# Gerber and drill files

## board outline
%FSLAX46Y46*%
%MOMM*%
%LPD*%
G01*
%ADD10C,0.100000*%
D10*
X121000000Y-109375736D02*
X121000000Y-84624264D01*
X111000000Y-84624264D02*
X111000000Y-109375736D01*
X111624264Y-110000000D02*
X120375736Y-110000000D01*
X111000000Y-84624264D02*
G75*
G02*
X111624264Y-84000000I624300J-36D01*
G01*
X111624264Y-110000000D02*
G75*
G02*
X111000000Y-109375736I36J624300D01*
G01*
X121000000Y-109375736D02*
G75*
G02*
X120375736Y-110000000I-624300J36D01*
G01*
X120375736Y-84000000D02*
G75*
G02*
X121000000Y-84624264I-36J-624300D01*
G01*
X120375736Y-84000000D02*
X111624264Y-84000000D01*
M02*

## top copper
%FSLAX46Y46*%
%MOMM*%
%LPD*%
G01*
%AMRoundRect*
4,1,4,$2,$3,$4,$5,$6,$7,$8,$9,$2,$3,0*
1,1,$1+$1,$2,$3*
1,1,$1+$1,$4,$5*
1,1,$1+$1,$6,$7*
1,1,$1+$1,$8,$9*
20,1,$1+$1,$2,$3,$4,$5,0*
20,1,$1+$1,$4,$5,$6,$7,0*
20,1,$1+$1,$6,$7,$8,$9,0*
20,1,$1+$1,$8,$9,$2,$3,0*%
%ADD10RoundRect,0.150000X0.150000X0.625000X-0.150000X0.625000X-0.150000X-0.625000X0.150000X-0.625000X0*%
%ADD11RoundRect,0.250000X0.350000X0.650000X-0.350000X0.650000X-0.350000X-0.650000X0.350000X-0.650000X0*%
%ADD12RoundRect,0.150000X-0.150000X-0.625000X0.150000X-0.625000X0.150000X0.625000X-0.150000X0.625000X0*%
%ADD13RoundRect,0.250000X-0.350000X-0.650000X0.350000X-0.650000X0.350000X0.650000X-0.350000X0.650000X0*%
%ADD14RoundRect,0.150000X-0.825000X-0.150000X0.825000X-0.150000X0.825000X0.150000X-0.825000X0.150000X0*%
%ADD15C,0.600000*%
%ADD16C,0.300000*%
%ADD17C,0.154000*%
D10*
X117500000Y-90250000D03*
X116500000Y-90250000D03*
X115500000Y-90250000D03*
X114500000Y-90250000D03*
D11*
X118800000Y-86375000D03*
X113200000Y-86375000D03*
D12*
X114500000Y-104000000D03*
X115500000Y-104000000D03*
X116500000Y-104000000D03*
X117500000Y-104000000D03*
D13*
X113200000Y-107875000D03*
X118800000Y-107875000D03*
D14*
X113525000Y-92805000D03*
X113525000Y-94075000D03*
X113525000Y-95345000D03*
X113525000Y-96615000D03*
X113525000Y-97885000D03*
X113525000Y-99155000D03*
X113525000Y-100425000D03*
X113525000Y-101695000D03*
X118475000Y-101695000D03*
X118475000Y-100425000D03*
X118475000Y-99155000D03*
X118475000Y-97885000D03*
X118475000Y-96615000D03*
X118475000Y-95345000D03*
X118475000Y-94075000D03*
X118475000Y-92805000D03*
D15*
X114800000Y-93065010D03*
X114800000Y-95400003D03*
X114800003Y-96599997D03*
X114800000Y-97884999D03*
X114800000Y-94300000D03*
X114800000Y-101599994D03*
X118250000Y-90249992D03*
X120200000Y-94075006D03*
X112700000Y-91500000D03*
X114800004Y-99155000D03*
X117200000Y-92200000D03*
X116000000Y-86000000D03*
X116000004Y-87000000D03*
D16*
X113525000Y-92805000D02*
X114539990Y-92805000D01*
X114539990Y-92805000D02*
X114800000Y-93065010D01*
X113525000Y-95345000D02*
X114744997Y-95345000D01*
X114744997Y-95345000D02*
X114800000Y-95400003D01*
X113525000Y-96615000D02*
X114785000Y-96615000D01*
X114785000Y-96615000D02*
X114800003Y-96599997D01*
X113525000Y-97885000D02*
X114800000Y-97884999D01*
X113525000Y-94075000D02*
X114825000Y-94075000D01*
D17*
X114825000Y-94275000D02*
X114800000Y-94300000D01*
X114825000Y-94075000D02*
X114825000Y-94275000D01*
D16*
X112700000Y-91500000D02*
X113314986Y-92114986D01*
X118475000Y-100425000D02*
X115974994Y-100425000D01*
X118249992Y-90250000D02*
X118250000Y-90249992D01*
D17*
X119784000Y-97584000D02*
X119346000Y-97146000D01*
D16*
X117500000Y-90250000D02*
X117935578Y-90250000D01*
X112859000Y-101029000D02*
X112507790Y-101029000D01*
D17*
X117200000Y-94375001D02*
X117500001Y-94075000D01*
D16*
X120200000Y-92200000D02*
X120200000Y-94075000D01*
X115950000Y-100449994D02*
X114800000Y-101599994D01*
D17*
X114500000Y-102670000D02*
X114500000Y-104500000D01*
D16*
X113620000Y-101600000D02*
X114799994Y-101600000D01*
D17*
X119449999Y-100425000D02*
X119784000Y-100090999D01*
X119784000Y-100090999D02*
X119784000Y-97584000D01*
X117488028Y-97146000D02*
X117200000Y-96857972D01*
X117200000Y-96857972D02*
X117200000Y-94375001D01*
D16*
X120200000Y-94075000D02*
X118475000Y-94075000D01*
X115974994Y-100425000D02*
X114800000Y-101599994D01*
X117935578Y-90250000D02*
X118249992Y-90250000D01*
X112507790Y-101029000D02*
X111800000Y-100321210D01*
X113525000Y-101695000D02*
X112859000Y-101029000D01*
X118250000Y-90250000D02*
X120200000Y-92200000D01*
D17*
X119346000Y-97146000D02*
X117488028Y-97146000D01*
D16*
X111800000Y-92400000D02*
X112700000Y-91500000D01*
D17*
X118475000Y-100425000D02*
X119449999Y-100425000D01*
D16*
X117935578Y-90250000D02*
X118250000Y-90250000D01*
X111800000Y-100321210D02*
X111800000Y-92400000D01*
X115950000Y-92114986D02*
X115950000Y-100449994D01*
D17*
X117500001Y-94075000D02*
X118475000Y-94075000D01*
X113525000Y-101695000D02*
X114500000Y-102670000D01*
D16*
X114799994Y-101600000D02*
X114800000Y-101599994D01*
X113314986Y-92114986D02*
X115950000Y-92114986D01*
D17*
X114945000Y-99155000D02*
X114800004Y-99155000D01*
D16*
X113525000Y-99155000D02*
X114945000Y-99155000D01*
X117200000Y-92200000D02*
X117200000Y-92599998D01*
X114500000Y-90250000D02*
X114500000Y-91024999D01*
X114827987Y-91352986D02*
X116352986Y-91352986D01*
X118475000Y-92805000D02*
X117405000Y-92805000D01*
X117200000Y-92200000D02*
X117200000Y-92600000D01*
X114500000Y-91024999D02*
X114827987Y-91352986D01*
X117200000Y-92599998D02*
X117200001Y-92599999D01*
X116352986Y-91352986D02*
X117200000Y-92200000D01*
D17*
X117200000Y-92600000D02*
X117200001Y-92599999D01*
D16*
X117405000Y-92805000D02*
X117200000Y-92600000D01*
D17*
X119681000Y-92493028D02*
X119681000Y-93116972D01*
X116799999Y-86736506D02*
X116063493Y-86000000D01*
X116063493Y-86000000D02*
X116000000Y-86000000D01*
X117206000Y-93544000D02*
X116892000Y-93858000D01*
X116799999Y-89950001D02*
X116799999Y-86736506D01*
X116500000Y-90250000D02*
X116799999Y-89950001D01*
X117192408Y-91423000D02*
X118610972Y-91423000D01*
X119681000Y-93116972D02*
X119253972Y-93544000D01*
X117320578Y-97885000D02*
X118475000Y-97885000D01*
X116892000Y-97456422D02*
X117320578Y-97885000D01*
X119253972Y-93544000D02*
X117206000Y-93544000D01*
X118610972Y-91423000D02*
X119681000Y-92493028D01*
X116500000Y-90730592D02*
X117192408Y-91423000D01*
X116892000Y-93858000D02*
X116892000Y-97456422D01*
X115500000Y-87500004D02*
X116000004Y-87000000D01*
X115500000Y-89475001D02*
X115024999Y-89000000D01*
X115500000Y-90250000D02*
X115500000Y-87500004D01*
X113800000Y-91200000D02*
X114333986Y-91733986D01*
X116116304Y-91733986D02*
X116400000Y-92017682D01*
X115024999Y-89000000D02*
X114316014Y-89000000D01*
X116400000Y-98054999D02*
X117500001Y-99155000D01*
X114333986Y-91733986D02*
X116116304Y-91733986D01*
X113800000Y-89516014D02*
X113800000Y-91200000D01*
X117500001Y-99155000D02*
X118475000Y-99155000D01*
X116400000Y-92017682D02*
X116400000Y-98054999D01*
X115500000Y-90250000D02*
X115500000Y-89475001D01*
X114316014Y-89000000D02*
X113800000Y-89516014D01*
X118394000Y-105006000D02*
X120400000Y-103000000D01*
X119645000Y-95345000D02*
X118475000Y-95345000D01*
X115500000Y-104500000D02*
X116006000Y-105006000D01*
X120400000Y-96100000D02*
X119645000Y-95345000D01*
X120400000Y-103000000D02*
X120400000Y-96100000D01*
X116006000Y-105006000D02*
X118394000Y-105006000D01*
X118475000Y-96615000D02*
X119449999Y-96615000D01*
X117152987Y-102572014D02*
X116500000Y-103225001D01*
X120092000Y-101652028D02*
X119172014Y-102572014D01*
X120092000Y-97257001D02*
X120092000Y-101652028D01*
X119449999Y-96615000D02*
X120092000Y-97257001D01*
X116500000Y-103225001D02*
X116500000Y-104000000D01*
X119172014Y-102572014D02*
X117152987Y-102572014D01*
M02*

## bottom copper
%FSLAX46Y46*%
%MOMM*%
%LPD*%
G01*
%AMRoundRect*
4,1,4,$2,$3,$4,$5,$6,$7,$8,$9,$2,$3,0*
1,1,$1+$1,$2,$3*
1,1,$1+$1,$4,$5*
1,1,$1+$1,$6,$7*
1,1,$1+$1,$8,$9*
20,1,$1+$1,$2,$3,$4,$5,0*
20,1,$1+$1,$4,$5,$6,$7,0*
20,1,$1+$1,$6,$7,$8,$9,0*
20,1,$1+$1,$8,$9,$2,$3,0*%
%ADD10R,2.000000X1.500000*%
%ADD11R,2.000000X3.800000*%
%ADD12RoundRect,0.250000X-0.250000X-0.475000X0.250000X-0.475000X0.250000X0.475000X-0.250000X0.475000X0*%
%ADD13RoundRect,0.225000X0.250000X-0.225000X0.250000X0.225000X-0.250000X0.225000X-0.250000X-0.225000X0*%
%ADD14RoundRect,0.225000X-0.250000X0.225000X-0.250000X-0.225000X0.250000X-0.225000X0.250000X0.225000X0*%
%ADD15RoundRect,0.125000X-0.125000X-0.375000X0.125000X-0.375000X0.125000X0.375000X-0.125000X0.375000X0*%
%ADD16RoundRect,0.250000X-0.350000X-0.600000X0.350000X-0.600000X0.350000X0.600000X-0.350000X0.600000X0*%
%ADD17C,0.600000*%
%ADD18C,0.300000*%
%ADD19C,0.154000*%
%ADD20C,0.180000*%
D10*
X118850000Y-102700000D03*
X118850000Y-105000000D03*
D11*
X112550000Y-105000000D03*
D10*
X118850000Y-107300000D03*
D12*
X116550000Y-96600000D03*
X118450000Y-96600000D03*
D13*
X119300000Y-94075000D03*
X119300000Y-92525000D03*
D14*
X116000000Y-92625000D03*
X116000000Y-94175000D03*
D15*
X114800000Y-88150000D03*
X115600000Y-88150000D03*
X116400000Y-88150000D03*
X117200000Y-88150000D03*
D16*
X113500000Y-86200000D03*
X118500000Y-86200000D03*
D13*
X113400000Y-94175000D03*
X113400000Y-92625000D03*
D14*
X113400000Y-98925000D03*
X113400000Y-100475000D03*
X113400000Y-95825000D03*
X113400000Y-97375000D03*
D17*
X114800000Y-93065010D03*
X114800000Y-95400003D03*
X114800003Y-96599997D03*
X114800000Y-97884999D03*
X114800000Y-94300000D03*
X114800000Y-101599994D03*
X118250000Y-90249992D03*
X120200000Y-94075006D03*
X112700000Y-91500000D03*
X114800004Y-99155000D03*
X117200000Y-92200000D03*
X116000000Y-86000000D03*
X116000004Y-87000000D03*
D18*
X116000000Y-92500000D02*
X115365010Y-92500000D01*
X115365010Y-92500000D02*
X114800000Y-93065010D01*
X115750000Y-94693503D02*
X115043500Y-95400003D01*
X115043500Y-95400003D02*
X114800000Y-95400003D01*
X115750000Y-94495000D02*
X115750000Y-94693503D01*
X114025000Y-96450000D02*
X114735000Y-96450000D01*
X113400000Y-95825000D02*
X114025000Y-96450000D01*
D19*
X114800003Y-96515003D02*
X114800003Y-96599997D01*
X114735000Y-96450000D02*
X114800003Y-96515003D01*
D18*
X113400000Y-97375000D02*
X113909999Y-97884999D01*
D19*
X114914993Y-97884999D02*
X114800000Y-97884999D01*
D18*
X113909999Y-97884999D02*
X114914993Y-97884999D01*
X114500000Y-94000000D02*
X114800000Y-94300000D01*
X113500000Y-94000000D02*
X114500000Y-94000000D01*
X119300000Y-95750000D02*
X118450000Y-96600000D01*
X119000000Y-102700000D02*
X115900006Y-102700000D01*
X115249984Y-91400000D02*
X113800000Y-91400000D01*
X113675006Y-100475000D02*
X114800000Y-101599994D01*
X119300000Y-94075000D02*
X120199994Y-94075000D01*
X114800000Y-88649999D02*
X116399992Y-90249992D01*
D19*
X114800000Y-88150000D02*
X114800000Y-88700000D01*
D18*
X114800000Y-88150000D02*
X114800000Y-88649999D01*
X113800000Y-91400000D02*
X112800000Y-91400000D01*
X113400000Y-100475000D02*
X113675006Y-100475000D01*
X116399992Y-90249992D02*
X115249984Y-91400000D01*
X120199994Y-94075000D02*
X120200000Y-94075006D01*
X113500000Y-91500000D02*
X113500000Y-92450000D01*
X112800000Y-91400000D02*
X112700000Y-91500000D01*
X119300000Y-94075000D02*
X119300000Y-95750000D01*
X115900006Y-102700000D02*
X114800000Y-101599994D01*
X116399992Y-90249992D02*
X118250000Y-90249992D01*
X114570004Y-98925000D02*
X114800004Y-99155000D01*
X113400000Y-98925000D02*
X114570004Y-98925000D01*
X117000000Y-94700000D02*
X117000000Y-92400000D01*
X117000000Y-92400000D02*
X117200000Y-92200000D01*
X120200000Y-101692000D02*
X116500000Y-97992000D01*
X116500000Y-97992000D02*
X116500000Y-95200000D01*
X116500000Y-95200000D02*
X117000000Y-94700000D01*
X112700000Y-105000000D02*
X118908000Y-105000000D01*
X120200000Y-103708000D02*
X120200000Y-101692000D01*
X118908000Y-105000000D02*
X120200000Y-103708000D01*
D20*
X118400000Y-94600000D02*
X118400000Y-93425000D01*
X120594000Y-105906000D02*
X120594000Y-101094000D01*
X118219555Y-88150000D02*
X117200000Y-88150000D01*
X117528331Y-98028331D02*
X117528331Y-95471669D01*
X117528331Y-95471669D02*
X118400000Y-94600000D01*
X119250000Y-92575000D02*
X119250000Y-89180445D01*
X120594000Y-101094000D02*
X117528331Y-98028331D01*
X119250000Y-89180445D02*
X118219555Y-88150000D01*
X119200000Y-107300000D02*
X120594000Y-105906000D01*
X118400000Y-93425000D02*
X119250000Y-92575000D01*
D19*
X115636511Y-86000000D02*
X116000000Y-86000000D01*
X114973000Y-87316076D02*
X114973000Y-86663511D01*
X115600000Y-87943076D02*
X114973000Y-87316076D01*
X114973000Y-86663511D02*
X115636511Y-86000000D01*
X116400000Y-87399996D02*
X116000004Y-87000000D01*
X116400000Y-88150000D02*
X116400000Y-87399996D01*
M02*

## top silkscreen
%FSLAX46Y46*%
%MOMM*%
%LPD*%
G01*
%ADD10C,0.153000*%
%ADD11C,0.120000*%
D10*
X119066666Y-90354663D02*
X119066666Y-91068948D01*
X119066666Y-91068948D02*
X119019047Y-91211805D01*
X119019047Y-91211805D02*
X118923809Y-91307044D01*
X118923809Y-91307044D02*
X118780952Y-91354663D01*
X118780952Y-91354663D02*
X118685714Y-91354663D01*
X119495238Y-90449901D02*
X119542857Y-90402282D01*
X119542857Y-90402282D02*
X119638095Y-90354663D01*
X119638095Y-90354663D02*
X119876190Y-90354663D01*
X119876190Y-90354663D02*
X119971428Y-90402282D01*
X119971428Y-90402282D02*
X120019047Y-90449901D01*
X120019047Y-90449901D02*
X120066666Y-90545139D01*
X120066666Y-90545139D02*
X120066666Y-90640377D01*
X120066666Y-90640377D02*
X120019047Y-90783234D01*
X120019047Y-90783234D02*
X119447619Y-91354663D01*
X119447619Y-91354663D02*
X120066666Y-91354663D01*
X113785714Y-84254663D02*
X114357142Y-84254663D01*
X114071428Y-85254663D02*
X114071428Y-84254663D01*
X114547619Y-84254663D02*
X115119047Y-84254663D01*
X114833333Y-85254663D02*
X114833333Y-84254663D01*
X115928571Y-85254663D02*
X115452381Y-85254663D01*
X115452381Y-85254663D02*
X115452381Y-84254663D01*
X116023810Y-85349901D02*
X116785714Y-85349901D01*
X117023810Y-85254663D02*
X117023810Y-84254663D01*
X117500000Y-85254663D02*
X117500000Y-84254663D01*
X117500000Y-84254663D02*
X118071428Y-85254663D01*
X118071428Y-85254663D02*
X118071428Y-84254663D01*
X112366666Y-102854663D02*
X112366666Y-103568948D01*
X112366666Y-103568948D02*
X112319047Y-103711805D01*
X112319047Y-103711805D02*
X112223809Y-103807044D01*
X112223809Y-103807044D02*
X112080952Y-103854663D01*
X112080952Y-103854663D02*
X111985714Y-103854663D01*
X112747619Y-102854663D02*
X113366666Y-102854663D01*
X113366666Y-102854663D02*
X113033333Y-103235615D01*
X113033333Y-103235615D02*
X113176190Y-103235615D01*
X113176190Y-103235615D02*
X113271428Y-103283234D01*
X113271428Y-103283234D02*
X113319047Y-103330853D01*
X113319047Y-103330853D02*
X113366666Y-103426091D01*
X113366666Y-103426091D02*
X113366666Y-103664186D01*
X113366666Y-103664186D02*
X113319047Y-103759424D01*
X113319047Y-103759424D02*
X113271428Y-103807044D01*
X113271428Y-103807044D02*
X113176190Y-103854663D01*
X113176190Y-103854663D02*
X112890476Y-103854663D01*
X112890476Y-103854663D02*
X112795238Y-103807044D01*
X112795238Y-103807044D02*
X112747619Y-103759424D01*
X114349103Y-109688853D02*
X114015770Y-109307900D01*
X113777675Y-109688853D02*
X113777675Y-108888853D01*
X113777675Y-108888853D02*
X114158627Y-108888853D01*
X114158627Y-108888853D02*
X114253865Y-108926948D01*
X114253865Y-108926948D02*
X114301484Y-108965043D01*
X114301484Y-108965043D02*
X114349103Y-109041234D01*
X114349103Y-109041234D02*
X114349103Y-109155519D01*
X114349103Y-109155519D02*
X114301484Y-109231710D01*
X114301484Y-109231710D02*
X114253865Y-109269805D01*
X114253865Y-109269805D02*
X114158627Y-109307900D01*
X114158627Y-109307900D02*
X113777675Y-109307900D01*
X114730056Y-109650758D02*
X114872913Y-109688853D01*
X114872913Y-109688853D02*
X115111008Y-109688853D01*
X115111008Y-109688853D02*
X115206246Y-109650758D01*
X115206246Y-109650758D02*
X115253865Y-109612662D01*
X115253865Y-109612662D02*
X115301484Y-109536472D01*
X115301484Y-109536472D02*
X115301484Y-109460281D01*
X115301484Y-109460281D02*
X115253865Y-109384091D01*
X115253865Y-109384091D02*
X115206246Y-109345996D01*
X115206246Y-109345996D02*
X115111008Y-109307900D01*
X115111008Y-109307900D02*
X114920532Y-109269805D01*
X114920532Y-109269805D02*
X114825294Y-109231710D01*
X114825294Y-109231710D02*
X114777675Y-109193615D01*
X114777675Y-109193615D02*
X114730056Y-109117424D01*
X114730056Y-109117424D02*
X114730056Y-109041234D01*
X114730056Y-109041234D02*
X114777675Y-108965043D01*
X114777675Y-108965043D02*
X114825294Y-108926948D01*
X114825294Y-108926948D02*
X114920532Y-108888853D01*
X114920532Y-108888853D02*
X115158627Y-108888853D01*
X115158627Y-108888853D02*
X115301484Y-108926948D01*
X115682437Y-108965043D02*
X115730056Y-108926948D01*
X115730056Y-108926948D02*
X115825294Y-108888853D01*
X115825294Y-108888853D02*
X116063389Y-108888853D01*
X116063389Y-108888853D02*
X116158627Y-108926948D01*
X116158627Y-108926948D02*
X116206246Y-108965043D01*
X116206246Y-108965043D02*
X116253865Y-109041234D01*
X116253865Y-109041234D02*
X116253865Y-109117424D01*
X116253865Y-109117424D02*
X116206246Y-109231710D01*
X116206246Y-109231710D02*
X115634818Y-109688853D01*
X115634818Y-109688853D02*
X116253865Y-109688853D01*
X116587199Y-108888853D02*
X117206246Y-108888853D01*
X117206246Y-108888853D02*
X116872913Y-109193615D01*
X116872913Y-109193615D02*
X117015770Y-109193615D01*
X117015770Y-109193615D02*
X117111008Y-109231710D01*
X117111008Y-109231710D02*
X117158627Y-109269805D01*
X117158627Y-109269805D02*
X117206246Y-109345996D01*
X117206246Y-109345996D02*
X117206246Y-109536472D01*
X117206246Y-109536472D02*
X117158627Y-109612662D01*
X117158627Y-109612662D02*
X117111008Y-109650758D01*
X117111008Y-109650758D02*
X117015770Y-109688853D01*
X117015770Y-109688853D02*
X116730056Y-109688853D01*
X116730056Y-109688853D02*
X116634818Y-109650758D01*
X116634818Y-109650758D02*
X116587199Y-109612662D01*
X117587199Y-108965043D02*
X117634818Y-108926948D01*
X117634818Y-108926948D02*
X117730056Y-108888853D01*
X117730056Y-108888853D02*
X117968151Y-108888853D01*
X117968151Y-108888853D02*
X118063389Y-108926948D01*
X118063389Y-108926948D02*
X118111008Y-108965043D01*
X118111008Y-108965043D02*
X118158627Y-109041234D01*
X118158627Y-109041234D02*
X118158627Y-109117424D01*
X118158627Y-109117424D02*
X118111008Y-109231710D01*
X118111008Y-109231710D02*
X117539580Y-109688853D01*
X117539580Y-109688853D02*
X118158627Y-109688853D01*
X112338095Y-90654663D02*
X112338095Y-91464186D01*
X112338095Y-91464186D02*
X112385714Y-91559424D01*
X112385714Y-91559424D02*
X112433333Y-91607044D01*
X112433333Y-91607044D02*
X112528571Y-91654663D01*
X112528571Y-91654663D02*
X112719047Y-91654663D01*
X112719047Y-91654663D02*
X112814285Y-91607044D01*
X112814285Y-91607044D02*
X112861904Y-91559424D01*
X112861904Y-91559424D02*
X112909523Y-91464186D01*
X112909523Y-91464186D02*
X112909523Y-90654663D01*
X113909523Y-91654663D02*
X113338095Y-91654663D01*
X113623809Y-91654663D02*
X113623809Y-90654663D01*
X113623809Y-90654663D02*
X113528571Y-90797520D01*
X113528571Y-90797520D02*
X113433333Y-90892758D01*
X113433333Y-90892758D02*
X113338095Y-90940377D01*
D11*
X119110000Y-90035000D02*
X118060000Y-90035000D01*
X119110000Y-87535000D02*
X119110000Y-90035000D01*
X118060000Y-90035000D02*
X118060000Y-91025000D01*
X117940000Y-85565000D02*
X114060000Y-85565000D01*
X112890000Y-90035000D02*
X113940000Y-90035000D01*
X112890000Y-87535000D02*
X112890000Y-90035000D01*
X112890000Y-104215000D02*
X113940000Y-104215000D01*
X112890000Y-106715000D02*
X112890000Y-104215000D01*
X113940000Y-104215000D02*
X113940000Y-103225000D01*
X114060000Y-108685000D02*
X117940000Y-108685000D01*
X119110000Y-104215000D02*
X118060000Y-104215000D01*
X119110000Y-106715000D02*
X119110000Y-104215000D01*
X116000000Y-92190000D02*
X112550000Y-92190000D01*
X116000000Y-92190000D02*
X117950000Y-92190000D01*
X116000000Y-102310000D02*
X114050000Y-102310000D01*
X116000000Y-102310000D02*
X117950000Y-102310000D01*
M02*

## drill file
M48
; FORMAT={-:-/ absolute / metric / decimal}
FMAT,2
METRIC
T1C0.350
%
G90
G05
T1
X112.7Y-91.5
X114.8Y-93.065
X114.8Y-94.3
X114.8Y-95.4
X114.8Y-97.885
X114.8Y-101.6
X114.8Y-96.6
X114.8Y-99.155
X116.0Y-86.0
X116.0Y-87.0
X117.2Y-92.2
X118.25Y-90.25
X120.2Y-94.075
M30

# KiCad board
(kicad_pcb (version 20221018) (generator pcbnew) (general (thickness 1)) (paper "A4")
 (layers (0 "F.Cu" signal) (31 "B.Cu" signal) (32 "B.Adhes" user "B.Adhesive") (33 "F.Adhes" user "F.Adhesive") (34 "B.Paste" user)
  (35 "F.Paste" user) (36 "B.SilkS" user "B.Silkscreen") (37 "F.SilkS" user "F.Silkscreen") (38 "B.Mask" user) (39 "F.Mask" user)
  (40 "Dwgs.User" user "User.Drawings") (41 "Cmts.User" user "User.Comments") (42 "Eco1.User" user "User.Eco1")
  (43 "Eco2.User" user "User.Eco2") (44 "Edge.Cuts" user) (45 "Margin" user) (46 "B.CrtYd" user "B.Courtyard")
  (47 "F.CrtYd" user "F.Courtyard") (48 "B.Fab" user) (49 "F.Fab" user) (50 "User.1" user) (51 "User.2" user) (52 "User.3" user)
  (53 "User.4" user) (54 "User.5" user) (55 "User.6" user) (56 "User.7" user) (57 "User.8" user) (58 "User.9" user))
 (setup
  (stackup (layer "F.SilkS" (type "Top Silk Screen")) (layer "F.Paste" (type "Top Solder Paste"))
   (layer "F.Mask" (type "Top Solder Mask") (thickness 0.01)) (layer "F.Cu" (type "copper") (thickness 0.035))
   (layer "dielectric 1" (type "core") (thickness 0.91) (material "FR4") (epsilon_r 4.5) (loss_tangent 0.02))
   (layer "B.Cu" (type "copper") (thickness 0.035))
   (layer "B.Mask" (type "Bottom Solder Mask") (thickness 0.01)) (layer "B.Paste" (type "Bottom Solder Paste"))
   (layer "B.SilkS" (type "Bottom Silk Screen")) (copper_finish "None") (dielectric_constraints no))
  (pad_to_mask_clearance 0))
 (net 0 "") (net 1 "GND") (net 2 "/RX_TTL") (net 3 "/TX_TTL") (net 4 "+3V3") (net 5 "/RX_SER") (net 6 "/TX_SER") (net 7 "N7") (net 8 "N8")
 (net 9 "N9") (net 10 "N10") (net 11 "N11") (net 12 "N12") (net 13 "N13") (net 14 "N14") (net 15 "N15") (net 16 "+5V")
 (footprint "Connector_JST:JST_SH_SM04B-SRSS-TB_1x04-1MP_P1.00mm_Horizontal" (layer "F.Cu") (at 116 88.25 180)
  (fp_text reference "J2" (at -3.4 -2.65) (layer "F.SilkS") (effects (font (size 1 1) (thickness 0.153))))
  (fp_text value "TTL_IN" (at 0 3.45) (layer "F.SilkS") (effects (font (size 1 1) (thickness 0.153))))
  (fp_line (start -3.11 -1.785) (end -2.06 -1.785) (stroke (width 0.12) (type solid)) (layer "F.SilkS"))
  (fp_line (start -3.11 0.715) (end -3.11 -1.785) (stroke (width 0.12) (type solid)) (layer "F.SilkS"))
  (fp_line (start -2.06 -1.785) (end -2.06 -2.775) (stroke (width 0.12) (type solid)) (layer "F.SilkS"))
  (fp_line (start -1.94 2.685) (end 1.94 2.685) (stroke (width 0.12) (type solid)) (layer "F.SilkS"))
  (fp_line (start 3.11 -1.785) (end 2.06 -1.785) (stroke (width 0.12) (type solid)) (layer "F.SilkS"))
  (fp_line (start 3.11 0.715) (end 3.11 -1.785) (stroke (width 0.12) (type solid)) (layer "F.SilkS"))
  (pad "1" smd roundrect (at -1.5 -2 180) (size 0.6 1.55) (layers "F.Cu" "F.Paste" "F.Mask") (roundrect_rratio 0.25) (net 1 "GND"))
  (pad "2" smd roundrect (at -0.5 -2 180) (size 0.6 1.55) (layers "F.Cu" "F.Paste" "F.Mask") (roundrect_rratio 0.25) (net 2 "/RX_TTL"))
  (pad "3" smd roundrect (at 0.5 -2 180) (size 0.6 1.55) (layers "F.Cu" "F.Paste" "F.Mask") (roundrect_rratio 0.25) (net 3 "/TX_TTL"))
  (pad "4" smd roundrect (at 1.5 -2 180) (size 0.6 1.55) (layers "F.Cu" "F.Paste" "F.Mask") (roundrect_rratio 0.25) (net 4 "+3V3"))
  (pad "MP" smd roundrect (at -2.8 1.875 180) (size 1.2 1.8) (layers "F.Cu" "F.Paste" "F.Mask") (roundrect_rratio 0.2083333333))
  (pad "MP" smd roundrect (at 2.8 1.875 180) (size 1.2 1.8) (layers "F.Cu" "F.Paste" "F.Mask") (roundrect_rratio 0.2083333333)))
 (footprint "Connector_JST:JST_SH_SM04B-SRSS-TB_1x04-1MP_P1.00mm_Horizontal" (layer "F.Cu") (at 116 106)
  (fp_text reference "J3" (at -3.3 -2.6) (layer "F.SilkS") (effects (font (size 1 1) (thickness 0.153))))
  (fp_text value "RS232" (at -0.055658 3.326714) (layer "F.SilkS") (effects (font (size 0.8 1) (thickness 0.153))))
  (fp_line (start -3.11 -1.785) (end -2.06 -1.785) (stroke (width 0.12) (type solid)) (layer "F.SilkS"))
  (fp_line (start -3.11 0.715) (end -3.11 -1.785) (stroke (width 0.12) (type solid)) (layer "F.SilkS"))
  (fp_line (start -2.06 -1.785) (end -2.06 -2.775) (stroke (width 0.12) (type solid)) (layer "F.SilkS"))
  (fp_line (start -1.94 2.685) (end 1.94 2.685) (stroke (width 0.12) (type solid)) (layer "F.SilkS"))
  (fp_line (start 3.11 -1.785) (end 2.06 -1.785) (stroke (width 0.12) (type solid)) (layer "F.SilkS"))
  (fp_line (start 3.11 0.715) (end 3.11 -1.785) (stroke (width 0.12) (type solid)) (layer "F.SilkS"))
  (pad "1" smd roundrect (at -1.5 -2) (size 0.6 1.55) (layers "F.Cu" "F.Paste" "F.Mask") (roundrect_rratio 0.25) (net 1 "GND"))
  (pad "2" smd roundrect (at -0.5 -2) (size 0.6 1.55) (layers "F.Cu" "F.Paste" "F.Mask") (roundrect_rratio 0.25) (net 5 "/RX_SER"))
  (pad "3" smd roundrect (at 0.5 -2) (size 0.6 1.55) (layers "F.Cu" "F.Paste" "F.Mask") (roundrect_rratio 0.25) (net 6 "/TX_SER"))
  (pad "4" smd roundrect (at 1.5 -2) (size 0.6 1.55) (layers "F.Cu" "F.Paste" "F.Mask") (roundrect_rratio 0.25) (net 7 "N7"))
  (pad "MP" smd roundrect (at -2.8 1.875) (size 1.2 1.8) (layers "F.Cu" "F.Paste" "F.Mask") (roundrect_rratio 0.2083333333))
  (pad "MP" smd roundrect (at 2.8 1.875) (size 1.2 1.8) (layers "F.Cu" "F.Paste" "F.Mask") (roundrect_rratio 0.2083333333)))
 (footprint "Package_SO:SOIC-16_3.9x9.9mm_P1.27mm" (layer "F.Cu") (at 116 97.25)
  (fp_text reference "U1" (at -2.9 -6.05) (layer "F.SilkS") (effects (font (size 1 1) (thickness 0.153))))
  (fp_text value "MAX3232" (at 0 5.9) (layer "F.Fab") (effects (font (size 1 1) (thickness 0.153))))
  (fp_line (start 0 -5.06) (end -3.45 -5.06) (stroke (width 0.12) (type solid)) (layer "F.SilkS"))
  (fp_line (start 0 -5.06) (end 1.95 -5.06) (stroke (width 0.12) (type solid)) (layer "F.SilkS"))
  (fp_line (start 0 5.06) (end -1.95 5.06) (stroke (width 0.12) (type solid)) (layer "F.SilkS"))
  (fp_line (start 0 5.06) (end 1.95 5.06) (stroke (width 0.12) (type solid)) (layer "F.SilkS"))
  (pad "1" smd roundrect (at -2.475 -4.445) (size 1.95 0.6) (layers "F.Cu" "F.Paste" "F.Mask") (roundrect_rratio 0.25) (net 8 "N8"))
  (pad "2" smd roundrect (at -2.475 -3.175) (size 1.95 0.6) (layers "F.Cu" "F.Paste" "F.Mask") (roundrect_rratio 0.25) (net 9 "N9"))
  (pad "3" smd roundrect (at -2.475 -1.905) (size 1.95 0.6) (layers "F.Cu" "F.Paste" "F.Mask") (roundrect_rratio 0.25) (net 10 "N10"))
  (pad "4" smd roundrect (at -2.475 -0.635) (size 1.95 0.6) (layers "F.Cu" "F.Paste" "F.Mask") (roundrect_rratio 0.25) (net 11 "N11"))
  (pad "5" smd roundrect (at -2.475 0.635) (size 1.95 0.6) (layers "F.Cu" "F.Paste" "F.Mask") (roundrect_rratio 0.25) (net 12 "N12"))
  (pad "6" smd roundrect (at -2.475 1.905) (size 1.95 0.6) (layers "F.Cu" "F.Paste" "F.Mask") (roundrect_rratio 0.25) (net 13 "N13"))
  (pad "7" smd roundrect (at -2.475 3.175) (size 1.95 0.6) (layers "F.Cu" "F.Paste" "F.Mask") (roundrect_rratio 0.25) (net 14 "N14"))
  (pad "8" smd roundrect (at -2.475 4.445) (size 1.95 0.6) (layers "F.Cu" "F.Paste" "F.Mask") (roundrect_rratio 0.25) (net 1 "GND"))
  (pad "9" smd roundrect (at 2.475 4.445) (size 1.95 0.6) (layers "F.Cu" "F.Paste" "F.Mask") (roundrect_rratio 0.25) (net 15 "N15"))
  (pad "10" smd roundrect (at 2.475 3.175) (size 1.95 0.6) (layers "F.Cu" "F.Paste" "F.Mask") (roundrect_rratio 0.25) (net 1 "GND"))
  (pad "11" smd roundrect (at 2.475 1.905) (size 1.95 0.6) (layers "F.Cu" "F.Paste" "F.Mask") (roundrect_rratio 0.25) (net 3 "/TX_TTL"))
  (pad "12" smd roundrect (at 2.475 0.635) (size 1.95 0.6) (layers "F.Cu" "F.Paste" "F.Mask") (roundrect_rratio 0.25) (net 2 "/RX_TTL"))
  (pad "13" smd roundrect (at 2.475 -0.635) (size 1.95 0.6) (layers "F.Cu" "F.Paste" "F.Mask") (roundrect_rratio 0.25) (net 6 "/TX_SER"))
  (pad "14" smd roundrect (at 2.475 -1.905) (size 1.95 0.6) (layers "F.Cu" "F.Paste" "F.Mask") (roundrect_rratio 0.25) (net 5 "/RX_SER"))
  (pad "15" smd roundrect (at 2.475 -3.175) (size 1.95 0.6) (layers "F.Cu" "F.Paste" "F.Mask") (roundrect_rratio 0.25) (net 1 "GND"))
  (pad "16" smd roundrect (at 2.475 -4.445) (size 1.95 0.6) (layers "F.Cu" "F.Paste" "F.Mask") (roundrect_rratio 0.25) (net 4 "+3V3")))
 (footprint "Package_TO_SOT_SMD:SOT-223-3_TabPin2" (layer "B.Cu") (at 115.7 105 180)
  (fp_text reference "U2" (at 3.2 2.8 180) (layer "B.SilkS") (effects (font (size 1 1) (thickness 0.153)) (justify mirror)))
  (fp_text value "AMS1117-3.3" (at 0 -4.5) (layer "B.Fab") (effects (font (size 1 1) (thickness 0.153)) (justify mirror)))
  (pad "1" smd rect (at -3.15 2.3 180) (size 2 1.5) (layers "B.Cu" "B.Paste" "B.Mask") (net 1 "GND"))
  (pad "2" smd rect (at -3.15 0 180) (size 2 1.5) (layers "B.Cu" "B.Paste" "B.Mask") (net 4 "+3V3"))
  (pad "2" smd rect (at 3.15 0 180) (size 2 3.8) (layers "B.Cu" "B.Paste" "B.Mask") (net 4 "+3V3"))
  (pad "3" smd rect (at -3.15 -2.3 180) (size 2 1.5) (layers "B.Cu" "B.Paste" "B.Mask") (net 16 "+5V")))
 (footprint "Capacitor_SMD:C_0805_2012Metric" (layer "B.Cu") (at 117.5 96.6)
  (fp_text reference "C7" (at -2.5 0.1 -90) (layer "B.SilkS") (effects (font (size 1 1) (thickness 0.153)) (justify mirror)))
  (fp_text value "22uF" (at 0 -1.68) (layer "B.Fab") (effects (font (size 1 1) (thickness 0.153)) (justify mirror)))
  (pad "1" smd roundrect (at -0.95 0) (size 1 1.45) (layers "B.Cu" "B.Paste" "B.Mask") (roundrect_rratio 0.25) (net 4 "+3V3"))
  (pad "2" smd roundrect (at 0.95 0) (size 1 1.45) (layers "B.Cu" "B.Paste" "B.Mask") (roundrect_rratio 0.25) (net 1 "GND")))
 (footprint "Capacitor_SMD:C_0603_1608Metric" (layer "B.Cu") (at 119.3 93.3 90)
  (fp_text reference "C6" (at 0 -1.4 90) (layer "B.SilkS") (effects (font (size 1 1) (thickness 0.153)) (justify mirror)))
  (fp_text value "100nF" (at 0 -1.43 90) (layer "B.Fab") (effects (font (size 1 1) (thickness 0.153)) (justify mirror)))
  (pad "1" smd roundrect (at -0.775 0 90) (size 0.9 0.95) (layers "B.Cu" "B.Paste" "B.Mask") (roundrect_rratio 0.25) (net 1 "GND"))
  (pad "2" smd roundrect (at 0.775 0 90) (size 0.9 0.95) (layers "B.Cu" "B.Paste" "B.Mask") (roundrect_rratio 0.25) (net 16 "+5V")))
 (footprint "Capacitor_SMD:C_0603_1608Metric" (layer "B.Cu") (at 116 93.4 -90)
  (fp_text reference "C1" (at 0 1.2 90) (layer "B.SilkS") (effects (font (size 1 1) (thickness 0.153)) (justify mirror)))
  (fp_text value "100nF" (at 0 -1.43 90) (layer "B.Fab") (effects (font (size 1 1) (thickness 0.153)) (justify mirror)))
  (pad "1" smd roundrect (at -0.775 0 270) (size 0.9 0.95) (layers "B.Cu" "B.Paste" "B.Mask") (roundrect_rratio 0.25) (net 8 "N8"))
  (pad "2" smd roundrect (at 0.775 0 270) (size 0.9 0.95) (layers "B.Cu" "B.Paste" "B.Mask") (roundrect_rratio 0.25) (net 10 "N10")))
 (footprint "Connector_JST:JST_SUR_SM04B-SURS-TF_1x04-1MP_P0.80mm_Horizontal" (layer "B.Cu") (at 116 87)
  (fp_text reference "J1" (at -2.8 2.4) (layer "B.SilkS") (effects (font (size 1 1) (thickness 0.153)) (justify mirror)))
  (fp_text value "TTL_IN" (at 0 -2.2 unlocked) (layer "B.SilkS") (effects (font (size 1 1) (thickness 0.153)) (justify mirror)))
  (pad "1" smd roundrect (at -1.2 1.15) (size 0.5 1) (layers "B.Cu" "B.Paste" "B.Mask") (roundrect_rratio 0.25) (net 1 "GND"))
  (pad "2" smd roundrect (at -0.4 1.15) (size 0.5 1) (layers "B.Cu" "B.Paste" "B.Mask") (roundrect_rratio 0.25) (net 2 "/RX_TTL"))
  (pad "3" smd roundrect (at 0.4 1.15) (size 0.5 1) (layers "B.Cu" "B.Paste" "B.Mask") (roundrect_rratio 0.25) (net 3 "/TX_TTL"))
  (pad "4" smd roundrect (at 1.2 1.15) (size 0.5 1) (layers "B.Cu" "B.Paste" "B.Mask") (roundrect_rratio 0.25) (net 16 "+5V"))
  (pad "MP" smd roundrect (at -2.5 -0.8) (size 1.2 1.7) (layers "B.Cu" "B.Paste" "B.Mask") (roundrect_rratio 0.2083333333))
  (pad "MP" smd roundrect (at 2.5 -0.8) (size 1.2 1.7) (layers "B.Cu" "B.Paste" "B.Mask") (roundrect_rratio 0.2083333333)))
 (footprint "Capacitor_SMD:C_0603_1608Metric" (layer "B.Cu") (at 113.4 93.4 90)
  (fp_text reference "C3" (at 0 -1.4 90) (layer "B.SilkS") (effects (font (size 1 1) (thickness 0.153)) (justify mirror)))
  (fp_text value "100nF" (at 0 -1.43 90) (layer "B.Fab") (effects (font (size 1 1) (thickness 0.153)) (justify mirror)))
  (pad "1" smd roundrect (at -0.775 0 90) (size 0.9 0.95) (layers "B.Cu" "B.Paste" "B.Mask") (roundrect_rratio 0.25) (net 9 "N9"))
  (pad "2" smd roundrect (at 0.775 0 90) (size 0.9 0.95) (layers "B.Cu" "B.Paste" "B.Mask") (roundrect_rratio 0.25) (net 1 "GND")))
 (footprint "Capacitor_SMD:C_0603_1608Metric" (layer "B.Cu") (at 113.4 99.7 -90)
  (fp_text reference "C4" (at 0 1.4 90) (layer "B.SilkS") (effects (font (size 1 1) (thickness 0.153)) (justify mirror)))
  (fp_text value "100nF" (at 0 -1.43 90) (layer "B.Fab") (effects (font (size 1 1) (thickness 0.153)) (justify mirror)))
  (pad "1" smd roundrect (at -0.775 0 270) (size 0.9 0.95) (layers "B.Cu" "B.Paste" "B.Mask") (roundrect_rratio 0.25) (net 13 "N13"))
  (pad "2" smd roundrect (at 0.775 0 270) (size 0.9 0.95) (layers "B.Cu" "B.Paste" "B.Mask") (roundrect_rratio 0.25) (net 1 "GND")))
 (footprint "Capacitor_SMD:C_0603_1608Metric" (layer "B.Cu") (at 113.4 96.6 -90)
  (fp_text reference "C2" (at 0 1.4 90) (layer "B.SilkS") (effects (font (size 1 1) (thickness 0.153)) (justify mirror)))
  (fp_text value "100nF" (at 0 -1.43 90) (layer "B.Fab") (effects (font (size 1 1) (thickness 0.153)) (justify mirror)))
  (pad "1" smd roundrect (at -0.775 0 270) (size 0.9 0.95) (layers "B.Cu" "B.Paste" "B.Mask") (roundrect_rratio 0.25) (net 11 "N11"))
  (pad "2" smd roundrect (at 0.775 0 270) (size 0.9 0.95) (layers "B.Cu" "B.Paste" "B.Mask") (roundrect_rratio 0.25) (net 12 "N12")))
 (gr_line (start 121 109.375736) (end 121 84.624264) (stroke (width 0.1) (type default)) (layer "Edge.Cuts"))
 (gr_line (start 111 84.624264) (end 111 109.375736) (stroke (width 0.1) (type default)) (layer "Edge.Cuts"))
 (gr_line (start 111.624264 110) (end 120.375736 110) (stroke (width 0.1) (type default)) (layer "Edge.Cuts"))
 (gr_arc (start 111 84.624264) (mid 111.182843 84.182843) (end 111.624264 84) (stroke (width 0.1) (type default)) (layer "Edge.Cuts"))
 (gr_arc (start 111.624264 110) (mid 111.182853 109.817147) (end 111 109.375736) (stroke (width 0.1) (type default)) (layer "Edge.Cuts"))
 (gr_arc (start 121 109.375736) (mid 120.817147 109.817147) (end 120.375736 110) (stroke (width 0.1) (type default)) (layer "Edge.Cuts"))
 (gr_arc (start 120.375736 84) (mid 120.817157 84.182843) (end 121 84.624264) (stroke (width 0.1) (type default)) (layer "Edge.Cuts"))
 (gr_line (start 120.375736 84) (end 111.624264 84) (stroke (width 0.1) (type default)) (layer "Edge.Cuts"))
 (segment (start 113.525 92.805) (end 114.53999 92.805) (width 0.3) (layer "F.Cu") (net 8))
 (segment (start 114.53999 92.805) (end 114.8 93.06501) (width 0.3) (layer "F.Cu") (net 8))
 (via (at 114.8 93.06501) (size 0.6) (drill 0.35) (layers "F.Cu" "B.Cu") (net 8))
 (segment (start 116 92.5) (end 115.36501 92.5) (width 0.3) (layer "B.Cu") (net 8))
 (segment (start 115.36501 92.5) (end 114.8 93.06501) (width 0.3) (layer "B.Cu") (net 8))
 (segment (start 113.525 95.345) (end 114.744997 95.345) (width 0.3) (layer "F.Cu") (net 10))
 (segment (start 114.744997 95.345) (end 114.8 95.400003) (width 0.3) (layer "F.Cu") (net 10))
 (via (at 114.8 95.400003) (size 0.6) (drill 0.35) (layers "F.Cu" "B.Cu") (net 10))
 (segment (start 115.75 94.693503) (end 115.0435 95.400003) (width 0.3) (layer "B.Cu") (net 10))
 (segment (start 115.0435 95.400003) (end 114.8 95.400003) (width 0.3) (layer "B.Cu") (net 10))
 (segment (start 115.75 94.495) (end 115.75 94.693503) (width 0.3) (layer "B.Cu") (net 10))
 (segment (start 113.525 96.615) (end 114.785 96.615) (width 0.3) (layer "F.Cu") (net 11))
 (segment (start 114.785 96.615) (end 114.800003 96.599997) (width 0.3) (layer "F.Cu") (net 11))
 (via (at 114.800003 96.599997) (size 0.6) (drill 0.35) (layers "F.Cu" "B.Cu") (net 11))
 (segment (start 114.025 96.45) (end 114.735 96.45) (width 0.3) (layer "B.Cu") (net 11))
 (segment (start 113.4 95.825) (end 114.025 96.45) (width 0.3) (layer "B.Cu") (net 11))
 (segment (start 114.800003 96.515003) (end 114.800003 96.599997) (width 0.154) (layer "B.Cu") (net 11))
 (segment (start 114.735 96.45) (end 114.800003 96.515003) (width 0.154) (layer "B.Cu") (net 11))
 (segment (start 113.525 97.885) (end 114.8 97.884999) (width 0.3) (layer "F.Cu") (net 12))
 (via (at 114.8 97.884999) (size 0.6) (drill 0.35) (layers "F.Cu" "B.Cu") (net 12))
 (segment (start 113.4 97.375) (end 113.909999 97.884999) (width 0.3) (layer "B.Cu") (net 12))
 (segment (start 114.914993 97.884999) (end 114.8 97.884999) (width 0.154) (layer "B.Cu") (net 12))
 (segment (start 113.909999 97.884999) (end 114.914993 97.884999) (width 0.3) (layer "B.Cu") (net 12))
 (segment (start 113.525 94.075) (end 114.825 94.075) (width 0.3) (layer "F.Cu") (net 9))
 (segment (start 114.825 94.275) (end 114.8 94.3) (width 0.154) (layer "F.Cu") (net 9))
 (segment (start 114.825 94.075) (end 114.825 94.275) (width 0.154) (layer "F.Cu") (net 9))
 (via (at 114.8 94.3) (size 0.6) (drill 0.35) (layers "F.Cu" "B.Cu") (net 9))
 (segment (start 114.5 94) (end 114.8 94.3) (width 0.3) (layer "B.Cu") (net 9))
 (segment (start 113.5 94) (end 114.5 94) (width 0.3) (layer "B.Cu") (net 9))
 (segment (start 112.7 91.5) (end 113.314986 92.114986) (width 0.3) (layer "F.Cu") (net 1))
 (segment (start 118.475 100.425) (end 115.974994 100.425) (width 0.3) (layer "F.Cu") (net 1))
 (segment (start 118.249992 90.25) (end 118.25 90.249992) (width 0.3) (layer "F.Cu") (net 1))
 (segment (start 119.784 97.584) (end 119.346 97.146) (width 0.154) (layer "F.Cu") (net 1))
 (segment (start 117.5 90.25) (end 117.935578 90.25) (width 0.3) (layer "F.Cu") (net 1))
 (segment (start 112.859 101.029) (end 112.50779 101.029) (width 0.3) (layer "F.Cu") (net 1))
 (segment (start 117.2 94.375001) (end 117.500001 94.075) (width 0.154) (layer "F.Cu") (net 1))
 (segment (start 120.2 92.2) (end 120.2 94.075) (width 0.3) (layer "F.Cu") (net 1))
 (segment (start 115.95 100.449994) (end 114.8 101.599994) (width 0.3) (layer "F.Cu") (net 1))
 (segment (start 114.5 102.67) (end 114.5 104.5) (width 0.154) (layer "F.Cu") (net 1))
 (segment (start 113.62 101.6) (end 114.799994 101.6) (width 0.3) (layer "F.Cu") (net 1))
 (segment (start 119.449999 100.425) (end 119.784 100.090999) (width 0.154) (layer "F.Cu") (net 1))
 (segment (start 119.784 100.090999) (end 119.784 97.584) (width 0.154) (layer "F.Cu") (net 1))
 (segment (start 117.488028 97.146) (end 117.2 96.857972) (width 0.154) (layer "F.Cu") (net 1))
 (segment (start 117.2 96.857972) (end 117.2 94.375001) (width 0.154) (layer "F.Cu") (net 1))
 (segment (start 120.2 94.075) (end 118.475 94.075) (width 0.3) (layer "F.Cu") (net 1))
 (segment (start 115.974994 100.425) (end 114.8 101.599994) (width 0.3) (layer "F.Cu") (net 1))
 (segment (start 117.935578 90.25) (end 118.249992 90.25) (width 0.3) (layer "F.Cu") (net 1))
 (segment (start 112.50779 101.029) (end 111.8 100.32121) (width 0.3) (layer "F.Cu") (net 1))
 (segment (start 113.525 101.695) (end 112.859 101.029) (width 0.3) (layer "F.Cu") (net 1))
 (segment (start 118.25 90.25) (end 120.2 92.2) (width 0.3) (layer "F.Cu") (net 1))
 (segment (start 119.346 97.146) (end 117.488028 97.146) (width 0.154) (layer "F.Cu") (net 1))
 (segment (start 111.8 92.4) (end 112.7 91.5) (width 0.3) (layer "F.Cu") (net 1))
 (segment (start 118.475 100.425) (end 119.449999 100.425) (width 0.154) (layer "F.Cu") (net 1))
 (segment (start 117.935578 90.25) (end 118.25 90.25) (width 0.3) (layer "F.Cu") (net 1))
 (segment (start 111.8 100.32121) (end 111.8 92.4) (width 0.3) (layer "F.Cu") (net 1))
 (segment (start 115.95 92.114986) (end 115.95 100.449994) (width 0.3) (layer "F.Cu") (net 1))
 (segment (start 117.500001 94.075) (end 118.475 94.075) (width 0.154) (layer "F.Cu") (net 1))
 (segment (start 113.525 101.695) (end 114.5 102.67) (width 0.154) (layer "F.Cu") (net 1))
 (segment (start 114.799994 101.6) (end 114.8 101.599994) (width 0.3) (layer "F.Cu") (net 1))
 (segment (start 113.314986 92.114986) (end 115.95 92.114986) (width 0.3) (layer "F.Cu") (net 1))
 (via (at 114.8 101.599994) (size 0.6) (drill 0.35) (layers "F.Cu" "B.Cu") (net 1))
 (via (at 118.25 90.249992) (size 0.6) (drill 0.35) (layers "F.Cu" "B.Cu") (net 1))
 (via (at 120.2 94.075006) (size 0.6) (drill 0.35) (layers "F.Cu" "B.Cu") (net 1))
 (via (at 112.7 91.5) (size 0.6) (drill 0.35) (layers "F.Cu" "B.Cu") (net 1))
 (segment (start 119.3 95.75) (end 118.45 96.6) (width 0.3) (layer "B.Cu") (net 1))
 (segment (start 119 102.7) (end 115.900006 102.7) (width 0.3) (layer "B.Cu") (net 1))
 (segment (start 115.249984 91.4) (end 113.8 91.4) (width 0.3) (layer "B.Cu") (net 1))
 (segment (start 113.675006 100.475) (end 114.8 101.599994) (width 0.3) (layer "B.Cu") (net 1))
 (segment (start 119.3 94.075) (end 120.199994 94.075) (width 0.3) (layer "B.Cu") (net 1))
 (segment (start 114.8 88.649999) (end 116.399992 90.249992) (width 0.3) (layer "B.Cu") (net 1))
 (segment (start 114.8 88.15) (end 114.8 88.7) (width 0.154) (layer "B.Cu") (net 1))
 (segment (start 114.8 88.15) (end 114.8 88.649999) (width 0.3) (layer "B.Cu") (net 1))
 (segment (start 113.8 91.4) (end 112.8 91.4) (width 0.3) (layer "B.Cu") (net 1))
 (segment (start 113.4 100.475) (end 113.675006 100.475) (width 0.3) (layer "B.Cu") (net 1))
 (segment (start 116.399992 90.249992) (end 115.249984 91.4) (width 0.3) (layer "B.Cu") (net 1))
 (segment (start 120.199994 94.075) (end 120.2 94.075006) (width 0.3) (layer "B.Cu") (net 1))
 (segment (start 113.5 91.5) (end 113.5 92.45) (width 0.3) (layer "B.Cu") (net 1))
 (segment (start 112.8 91.4) (end 112.7 91.5) (width 0.3) (layer "B.Cu") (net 1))
 (segment (start 119.3 94.075) (end 119.3 95.75) (width 0.3) (layer "B.Cu") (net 1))
 (segment (start 115.900006 102.7) (end 114.8 101.599994) (width 0.3) (layer "B.Cu") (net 1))
 (segment (start 116.399992 90.249992) (end 118.25 90.249992) (width 0.3) (layer "B.Cu") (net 1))
 (segment (start 114.945 99.155) (end 114.800004 99.155) (width 0.154) (layer "F.Cu") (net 13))
 (segment (start 113.525 99.155) (end 114.945 99.155) (width 0.3) (layer "F.Cu") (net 13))
 (via (at 114.800004 99.155) (size 0.6) (drill 0.35) (layers "F.Cu" "B.Cu") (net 13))
 (segment (start 114.570004 98.925) (end 114.800004 99.155) (width 0.3) (layer "B.Cu") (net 13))
 (segment (start 113.4 98.925) (end 114.570004 98.925) (width 0.3) (layer "B.Cu") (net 13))
 (segment (start 117.2 92.2) (end 117.2 92.599998) (width 0.3) (layer "F.Cu") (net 4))
 (segment (start 114.5 90.25) (end 114.5 91.024999) (width 0.3) (layer "F.Cu") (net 4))
 (segment (start 114.827987 91.352986) (end 116.352986 91.352986) (width 0.3) (layer "F.Cu") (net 4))
 (segment (start 118.475 92.805) (end 117.405 92.805) (width 0.3) (layer "F.Cu") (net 4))
 (segment (start 117.2 92.2) (end 117.2 92.6) (width 0.3) (layer "F.Cu") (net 4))
 (segment (start 114.5 91.024999) (end 114.827987 91.352986) (width 0.3) (layer "F.Cu") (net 4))
 (segment (start 117.2 92.599998) (end 117.200001 92.599999) (width 0.3) (layer "F.Cu") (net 4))
 (segment (start 116.352986 91.352986) (end 117.2 92.2) (width 0.3) (layer "F.Cu") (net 4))
 (segment (start 117.2 92.6) (end 117.200001 92.599999) (width 0.154) (layer "F.Cu") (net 4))
 (segment (start 117.405 92.805) (end 117.2 92.6) (width 0.3) (layer "F.Cu") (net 4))
 (via (at 117.2 92.2) (size 0.6) (drill 0.35) (layers "F.Cu" "B.Cu") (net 4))
 (segment (start 117 94.7) (end 117 92.4) (width 0.3) (layer "B.Cu") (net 4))
 (segment (start 117 92.4) (end 117.2 92.2) (width 0.3) (layer "B.Cu") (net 4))
 (segment (start 120.2 101.692) (end 116.5 97.992) (width 0.3) (layer "B.Cu") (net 4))
 (segment (start 116.5 97.992) (end 116.5 95.2) (width 0.3) (layer "B.Cu") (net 4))
 (segment (start 116.5 95.2) (end 117 94.7) (width 0.3) (layer "B.Cu") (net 4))
 (segment (start 112.7 105) (end 118.908 105) (width 0.3) (layer "B.Cu") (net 4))
 (segment (start 120.2 103.708) (end 120.2 101.692) (width 0.3) (layer "B.Cu") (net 4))
 (segment (start 118.908 105) (end 120.2 103.708) (width 0.3) (layer "B.Cu") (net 4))
 (segment (start 118.4 94.6) (end 118.4 93.425) (width 0.18) (layer "B.Cu") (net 16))
 (segment (start 120.594 105.906) (end 120.594 101.094) (width 0.18) (layer "B.Cu") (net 16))
 (segment (start 118.219555 88.15) (end 117.2 88.15) (width 0.18) (layer "B.Cu") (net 16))
 (segment (start 117.528331 98.028331) (end 117.528331 95.471669) (width 0.18) (layer "B.Cu") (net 16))
 (segment (start 117.528331 95.471669) (end 118.4 94.6) (width 0.18) (layer "B.Cu") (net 16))
 (segment (start 119.25 92.575) (end 119.25 89.180445) (width 0.18) (layer "B.Cu") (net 16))
 (segment (start 120.594 101.094) (end 117.528331 98.028331) (width 0.18) (layer "B.Cu") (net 16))
 (segment (start 119.25 89.180445) (end 118.219555 88.15) (width 0.18) (layer "B.Cu") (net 16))
 (segment (start 119.2 107.3) (end 120.594 105.906) (width 0.18) (layer "B.Cu") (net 16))
 (segment (start 118.4 93.425) (end 119.25 92.575) (width 0.18) (layer "B.Cu") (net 16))
 (segment (start 119.681 92.493028) (end 119.681 93.116972) (width 0.154) (layer "F.Cu") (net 2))
 (segment (start 116.799999 86.736506) (end 116.063493 86) (width 0.154) (layer "F.Cu") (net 2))
 (segment (start 116.063493 86) (end 116 86) (width 0.154) (layer "F.Cu") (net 2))
 (segment (start 117.206 93.544) (end 116.892 93.858) (width 0.154) (layer "F.Cu") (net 2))
 (segment (start 116.799999 89.950001) (end 116.799999 86.736506) (width 0.154) (layer "F.Cu") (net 2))
 (segment (start 116.5 90.25) (end 116.799999 89.950001) (width 0.154) (layer "F.Cu") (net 2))
 (segment (start 117.192408 91.423) (end 118.610972 91.423) (width 0.154) (layer "F.Cu") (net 2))
 (segment (start 119.681 93.116972) (end 119.253972 93.544) (width 0.154) (layer "F.Cu") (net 2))
 (segment (start 117.320578 97.885) (end 118.475 97.885) (width 0.154) (layer "F.Cu") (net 2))
 (segment (start 116.892 97.456422) (end 117.320578 97.885) (width 0.154) (layer "F.Cu") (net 2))
 (segment (start 119.253972 93.544) (end 117.206 93.544) (width 0.154) (layer "F.Cu") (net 2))
 (segment (start 118.610972 91.423) (end 119.681 92.493028) (width 0.154) (layer "F.Cu") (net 2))
 (segment (start 116.5 90.730592) (end 117.192408 91.423) (width 0.154) (layer "F.Cu") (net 2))
 (segment (start 116.892 93.858) (end 116.892 97.456422) (width 0.154) (layer "F.Cu") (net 2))
 (via (at 116 86) (size 0.6) (drill 0.35) (layers "F.Cu" "B.Cu") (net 2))
 (segment (start 115.636511 86) (end 116 86) (width 0.154) (layer "B.Cu") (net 2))
 (segment (start 114.973 87.316076) (end 114.973 86.663511) (width 0.154) (layer "B.Cu") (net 2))
 (segment (start 115.6 87.943076) (end 114.973 87.316076) (width 0.154) (layer "B.Cu") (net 2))
 (segment (start 114.973 86.663511) (end 115.636511 86) (width 0.154) (layer "B.Cu") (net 2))
 (segment (start 115.5 87.500004) (end 116.000004 87) (width 0.154) (layer "F.Cu") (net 3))
 (segment (start 115.5 89.475001) (end 115.024999 89) (width 0.154) (layer "F.Cu") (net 3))
 (segment (start 115.5 90.25) (end 115.5 87.500004) (width 0.154) (layer "F.Cu") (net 3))
 (segment (start 113.8 91.2) (end 114.333986 91.733986) (width 0.154) (layer "F.Cu") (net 3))
 (segment (start 116.116304 91.733986) (end 116.4 92.017682) (width 0.154) (layer "F.Cu") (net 3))
 (segment (start 115.024999 89) (end 114.316014 89) (width 0.154) (layer "F.Cu") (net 3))
 (segment (start 116.4 98.054999) (end 117.500001 99.155) (width 0.154) (layer "F.Cu") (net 3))
 (segment (start 114.333986 91.733986) (end 116.116304 91.733986) (width 0.154) (layer "F.Cu") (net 3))
 (segment (start 113.8 89.516014) (end 113.8 91.2) (width 0.154) (layer "F.Cu") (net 3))
 (segment (start 117.500001 99.155) (end 118.475 99.155) (width 0.154) (layer "F.Cu") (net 3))
 (segment (start 116.4 92.017682) (end 116.4 98.054999) (width 0.154) (layer "F.Cu") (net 3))
 (segment (start 115.5 90.25) (end 115.5 89.475001) (width 0.154) (layer "F.Cu") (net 3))
 (segment (start 114.316014 89) (end 113.8 89.516014) (width 0.154) (layer "F.Cu") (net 3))
 (via (at 116.000004 87) (size 0.6) (drill 0.35) (layers "F.Cu" "B.Cu") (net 3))
 (segment (start 116.4 87.399996) (end 116.000004 87) (width 0.154) (layer "B.Cu") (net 3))
 (segment (start 116.4 88.15) (end 116.4 87.399996) (width 0.154) (layer "B.Cu") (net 3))
 (segment (start 118.394 105.006) (end 120.4 103) (width 0.154) (layer "F.Cu") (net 5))
 (segment (start 119.645 95.345) (end 118.475 95.345) (width 0.154) (layer "F.Cu") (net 5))
 (segment (start 115.5 104.5) (end 116.006 105.006) (width 0.154) (layer "F.Cu") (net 5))
 (segment (start 120.4 96.1) (end 119.645 95.345) (width 0.154) (layer "F.Cu") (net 5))
 (segment (start 120.4 103) (end 120.4 96.1) (width 0.154) (layer "F.Cu") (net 5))
 (segment (start 116.006 105.006) (end 118.394 105.006) (width 0.154) (layer "F.Cu") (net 5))
 (segment (start 118.475 96.615) (end 119.449999 96.615) (width 0.154) (layer "F.Cu") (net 6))
 (segment (start 117.152987 102.572014) (end 116.5 103.225001) (width 0.154) (layer "F.Cu") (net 6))
 (segment (start 120.092 101.652028) (end 119.172014 102.572014) (width 0.154) (layer "F.Cu") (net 6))
 (segment (start 120.092 97.257001) (end 120.092 101.652028) (width 0.154) (layer "F.Cu") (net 6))
 (segment (start 119.449999 96.615) (end 120.092 97.257001) (width 0.154) (layer "F.Cu") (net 6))
 (segment (start 116.5 103.225001) (end 116.5 104) (width 0.154) (layer "F.Cu") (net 6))
 (segment (start 119.172014 102.572014) (end 117.152987 102.572014) (width 0.154) (layer "F.Cu") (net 6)))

